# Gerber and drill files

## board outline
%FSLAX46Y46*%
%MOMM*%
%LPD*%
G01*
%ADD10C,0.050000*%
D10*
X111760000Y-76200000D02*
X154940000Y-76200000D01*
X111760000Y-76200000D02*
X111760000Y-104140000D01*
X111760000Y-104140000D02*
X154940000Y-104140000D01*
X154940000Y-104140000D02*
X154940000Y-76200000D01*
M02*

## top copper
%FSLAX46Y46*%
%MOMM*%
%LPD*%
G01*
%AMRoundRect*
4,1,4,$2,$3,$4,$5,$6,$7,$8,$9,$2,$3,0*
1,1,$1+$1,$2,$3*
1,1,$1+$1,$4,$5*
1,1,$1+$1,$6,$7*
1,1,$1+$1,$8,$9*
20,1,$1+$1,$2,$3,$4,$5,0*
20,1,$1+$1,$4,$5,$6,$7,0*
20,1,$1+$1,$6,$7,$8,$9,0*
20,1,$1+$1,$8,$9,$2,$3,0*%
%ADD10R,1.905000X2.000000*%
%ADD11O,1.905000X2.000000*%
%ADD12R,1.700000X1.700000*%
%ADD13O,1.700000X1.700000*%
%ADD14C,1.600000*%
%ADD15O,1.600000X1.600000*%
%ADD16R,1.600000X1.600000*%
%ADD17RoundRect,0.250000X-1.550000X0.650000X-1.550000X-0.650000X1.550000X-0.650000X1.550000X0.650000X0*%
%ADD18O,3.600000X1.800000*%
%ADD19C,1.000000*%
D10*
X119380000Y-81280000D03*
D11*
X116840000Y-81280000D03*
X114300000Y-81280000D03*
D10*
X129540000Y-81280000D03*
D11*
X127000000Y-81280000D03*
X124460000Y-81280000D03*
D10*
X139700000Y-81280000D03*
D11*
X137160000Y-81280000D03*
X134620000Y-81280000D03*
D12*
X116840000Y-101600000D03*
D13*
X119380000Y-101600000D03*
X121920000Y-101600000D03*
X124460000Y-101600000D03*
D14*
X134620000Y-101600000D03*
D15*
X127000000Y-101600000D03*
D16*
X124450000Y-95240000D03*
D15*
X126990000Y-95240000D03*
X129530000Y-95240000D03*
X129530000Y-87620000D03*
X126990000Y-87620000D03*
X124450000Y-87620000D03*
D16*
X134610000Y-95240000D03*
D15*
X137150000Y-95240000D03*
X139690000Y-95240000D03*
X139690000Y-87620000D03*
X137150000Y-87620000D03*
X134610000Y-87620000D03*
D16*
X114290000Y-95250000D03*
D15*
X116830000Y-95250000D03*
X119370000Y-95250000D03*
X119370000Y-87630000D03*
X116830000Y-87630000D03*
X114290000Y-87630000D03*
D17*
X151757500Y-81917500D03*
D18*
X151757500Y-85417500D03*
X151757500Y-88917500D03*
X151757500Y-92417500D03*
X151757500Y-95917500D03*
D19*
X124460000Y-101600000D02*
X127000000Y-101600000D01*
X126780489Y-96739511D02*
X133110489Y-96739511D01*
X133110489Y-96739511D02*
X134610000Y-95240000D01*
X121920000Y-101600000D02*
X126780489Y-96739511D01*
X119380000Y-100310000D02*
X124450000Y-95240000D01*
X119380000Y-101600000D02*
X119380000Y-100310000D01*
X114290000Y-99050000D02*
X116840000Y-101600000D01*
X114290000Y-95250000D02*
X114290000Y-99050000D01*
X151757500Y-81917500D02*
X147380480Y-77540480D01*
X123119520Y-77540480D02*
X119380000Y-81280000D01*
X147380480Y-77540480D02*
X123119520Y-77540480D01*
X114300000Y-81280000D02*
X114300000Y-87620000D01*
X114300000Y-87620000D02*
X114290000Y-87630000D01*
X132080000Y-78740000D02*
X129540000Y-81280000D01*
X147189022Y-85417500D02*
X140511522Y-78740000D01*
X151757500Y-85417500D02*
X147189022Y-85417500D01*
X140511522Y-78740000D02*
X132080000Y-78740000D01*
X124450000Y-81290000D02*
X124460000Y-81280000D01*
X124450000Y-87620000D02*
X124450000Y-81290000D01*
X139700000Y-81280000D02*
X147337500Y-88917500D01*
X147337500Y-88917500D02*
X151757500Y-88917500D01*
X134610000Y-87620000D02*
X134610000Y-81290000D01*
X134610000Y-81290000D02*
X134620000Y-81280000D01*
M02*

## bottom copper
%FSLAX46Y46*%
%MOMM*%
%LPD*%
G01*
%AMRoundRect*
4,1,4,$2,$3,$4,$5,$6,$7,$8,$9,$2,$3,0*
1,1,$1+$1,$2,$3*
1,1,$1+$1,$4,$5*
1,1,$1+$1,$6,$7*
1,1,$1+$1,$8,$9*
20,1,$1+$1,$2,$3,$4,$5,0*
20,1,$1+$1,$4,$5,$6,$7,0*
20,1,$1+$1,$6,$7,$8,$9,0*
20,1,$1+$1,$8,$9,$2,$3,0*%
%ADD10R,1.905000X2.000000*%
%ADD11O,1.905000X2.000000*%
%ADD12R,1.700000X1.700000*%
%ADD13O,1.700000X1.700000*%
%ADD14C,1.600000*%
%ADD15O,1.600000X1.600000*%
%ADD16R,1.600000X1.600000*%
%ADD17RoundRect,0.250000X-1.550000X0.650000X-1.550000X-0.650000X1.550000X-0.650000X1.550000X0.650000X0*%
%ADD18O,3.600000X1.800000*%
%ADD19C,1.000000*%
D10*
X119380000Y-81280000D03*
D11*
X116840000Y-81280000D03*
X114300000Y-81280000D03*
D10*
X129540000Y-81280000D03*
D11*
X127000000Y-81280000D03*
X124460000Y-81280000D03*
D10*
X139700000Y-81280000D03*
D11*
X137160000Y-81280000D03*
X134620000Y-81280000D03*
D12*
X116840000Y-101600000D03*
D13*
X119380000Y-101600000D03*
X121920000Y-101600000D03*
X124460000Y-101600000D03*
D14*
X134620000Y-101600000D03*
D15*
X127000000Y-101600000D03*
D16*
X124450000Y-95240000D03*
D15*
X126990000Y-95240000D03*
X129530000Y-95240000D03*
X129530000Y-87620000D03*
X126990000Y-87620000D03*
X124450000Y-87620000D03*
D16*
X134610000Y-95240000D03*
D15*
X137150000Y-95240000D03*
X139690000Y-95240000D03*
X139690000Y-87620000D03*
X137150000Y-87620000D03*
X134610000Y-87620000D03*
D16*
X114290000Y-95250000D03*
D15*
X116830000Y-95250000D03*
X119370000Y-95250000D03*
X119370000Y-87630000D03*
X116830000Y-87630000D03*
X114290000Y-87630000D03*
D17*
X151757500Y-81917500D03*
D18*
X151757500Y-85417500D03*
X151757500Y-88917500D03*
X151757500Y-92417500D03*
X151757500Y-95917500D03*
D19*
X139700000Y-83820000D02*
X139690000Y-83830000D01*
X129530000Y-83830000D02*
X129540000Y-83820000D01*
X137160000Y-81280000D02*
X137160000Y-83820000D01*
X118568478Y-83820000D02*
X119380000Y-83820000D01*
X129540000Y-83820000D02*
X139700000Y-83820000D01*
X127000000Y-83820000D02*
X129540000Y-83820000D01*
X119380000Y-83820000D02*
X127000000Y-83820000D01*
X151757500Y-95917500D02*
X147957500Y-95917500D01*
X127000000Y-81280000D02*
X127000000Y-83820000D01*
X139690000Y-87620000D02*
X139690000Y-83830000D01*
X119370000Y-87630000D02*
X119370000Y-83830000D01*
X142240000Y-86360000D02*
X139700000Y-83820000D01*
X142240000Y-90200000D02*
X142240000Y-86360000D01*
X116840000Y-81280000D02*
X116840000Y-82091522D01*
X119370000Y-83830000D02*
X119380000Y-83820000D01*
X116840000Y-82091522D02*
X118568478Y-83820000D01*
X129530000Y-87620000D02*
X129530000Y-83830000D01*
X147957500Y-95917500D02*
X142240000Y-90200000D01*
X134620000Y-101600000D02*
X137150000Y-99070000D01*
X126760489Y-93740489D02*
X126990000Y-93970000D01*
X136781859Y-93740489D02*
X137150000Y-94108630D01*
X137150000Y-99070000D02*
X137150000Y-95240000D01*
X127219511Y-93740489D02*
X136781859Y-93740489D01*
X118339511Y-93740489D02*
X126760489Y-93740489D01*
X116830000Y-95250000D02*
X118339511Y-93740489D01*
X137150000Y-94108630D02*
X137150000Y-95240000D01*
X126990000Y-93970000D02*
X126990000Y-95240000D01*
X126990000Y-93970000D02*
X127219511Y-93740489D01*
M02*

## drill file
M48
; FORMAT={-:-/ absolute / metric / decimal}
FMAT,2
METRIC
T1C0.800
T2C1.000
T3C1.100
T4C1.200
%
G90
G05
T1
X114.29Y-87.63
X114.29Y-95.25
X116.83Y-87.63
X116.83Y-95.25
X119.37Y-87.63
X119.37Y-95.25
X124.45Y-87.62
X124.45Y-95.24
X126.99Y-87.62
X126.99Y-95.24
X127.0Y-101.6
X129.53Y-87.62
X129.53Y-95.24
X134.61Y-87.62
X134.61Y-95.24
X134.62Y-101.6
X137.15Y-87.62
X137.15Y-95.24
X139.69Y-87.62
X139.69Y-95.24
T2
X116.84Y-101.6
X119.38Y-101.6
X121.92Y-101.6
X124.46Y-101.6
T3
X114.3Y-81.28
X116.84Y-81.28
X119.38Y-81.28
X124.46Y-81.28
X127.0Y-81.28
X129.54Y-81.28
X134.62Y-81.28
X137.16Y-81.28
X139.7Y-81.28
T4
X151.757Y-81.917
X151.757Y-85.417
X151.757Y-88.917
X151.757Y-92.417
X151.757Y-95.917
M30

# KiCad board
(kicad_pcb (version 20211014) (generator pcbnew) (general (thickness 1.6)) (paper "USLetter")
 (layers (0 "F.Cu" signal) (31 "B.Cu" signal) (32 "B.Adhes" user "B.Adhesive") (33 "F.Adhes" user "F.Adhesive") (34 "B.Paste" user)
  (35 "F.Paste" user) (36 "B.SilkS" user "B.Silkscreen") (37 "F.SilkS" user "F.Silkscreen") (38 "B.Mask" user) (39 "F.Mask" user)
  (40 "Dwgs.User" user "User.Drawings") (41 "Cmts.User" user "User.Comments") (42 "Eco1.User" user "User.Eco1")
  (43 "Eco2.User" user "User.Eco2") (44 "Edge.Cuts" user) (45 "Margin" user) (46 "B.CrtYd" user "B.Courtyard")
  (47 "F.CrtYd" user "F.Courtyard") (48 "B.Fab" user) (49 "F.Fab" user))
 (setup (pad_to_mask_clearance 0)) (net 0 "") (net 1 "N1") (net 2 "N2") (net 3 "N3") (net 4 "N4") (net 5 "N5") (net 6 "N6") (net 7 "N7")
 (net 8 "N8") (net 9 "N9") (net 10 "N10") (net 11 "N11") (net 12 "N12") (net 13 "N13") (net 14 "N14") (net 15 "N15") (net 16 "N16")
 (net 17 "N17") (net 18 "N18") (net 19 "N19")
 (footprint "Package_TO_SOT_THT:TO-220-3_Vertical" (layer "F.Cu") (at 119.38 81.28 180)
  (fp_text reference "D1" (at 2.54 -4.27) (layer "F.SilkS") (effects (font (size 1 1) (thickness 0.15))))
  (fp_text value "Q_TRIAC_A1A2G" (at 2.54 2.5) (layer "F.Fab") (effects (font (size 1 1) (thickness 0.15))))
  (pad "1" thru_hole rect locked (at 0 0 180) (size 1.905 2) (drill 1.1) (layers *.Cu *.Mask) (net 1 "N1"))
  (pad "2" thru_hole oval locked (at 2.54 0 180) (size 1.905 2) (drill 1.1) (layers *.Cu *.Mask) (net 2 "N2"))
  (pad "3" thru_hole oval locked (at 5.08 0 180) (size 1.905 2) (drill 1.1) (layers *.Cu *.Mask) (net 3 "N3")))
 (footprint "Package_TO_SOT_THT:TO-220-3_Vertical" (layer "F.Cu") (at 129.54 81.28 180)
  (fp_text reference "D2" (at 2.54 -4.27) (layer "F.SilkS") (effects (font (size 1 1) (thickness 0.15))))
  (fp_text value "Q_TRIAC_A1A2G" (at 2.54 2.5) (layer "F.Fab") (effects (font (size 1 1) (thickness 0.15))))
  (pad "1" thru_hole rect locked (at 0 0 180) (size 1.905 2) (drill 1.1) (layers *.Cu *.Mask) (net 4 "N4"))
  (pad "2" thru_hole oval locked (at 2.54 0 180) (size 1.905 2) (drill 1.1) (layers *.Cu *.Mask) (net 2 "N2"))
  (pad "3" thru_hole oval locked (at 5.08 0 180) (size 1.905 2) (drill 1.1) (layers *.Cu *.Mask) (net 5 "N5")))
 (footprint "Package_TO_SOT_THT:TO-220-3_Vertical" (layer "F.Cu") (at 139.7 81.28 180)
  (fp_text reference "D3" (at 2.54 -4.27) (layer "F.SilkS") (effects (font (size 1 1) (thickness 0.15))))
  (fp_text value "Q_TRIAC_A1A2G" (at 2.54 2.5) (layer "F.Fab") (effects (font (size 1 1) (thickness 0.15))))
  (pad "1" thru_hole rect locked (at 0 0 180) (size 1.905 2) (drill 1.1) (layers *.Cu *.Mask) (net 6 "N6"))
  (pad "2" thru_hole oval locked (at 2.54 0 180) (size 1.905 2) (drill 1.1) (layers *.Cu *.Mask) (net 2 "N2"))
  (pad "3" thru_hole oval locked (at 5.08 0 180) (size 1.905 2) (drill 1.1) (layers *.Cu *.Mask) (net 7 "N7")))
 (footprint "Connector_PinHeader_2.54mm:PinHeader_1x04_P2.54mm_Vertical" (layer "F.Cu") (at 116.84 101.6 90)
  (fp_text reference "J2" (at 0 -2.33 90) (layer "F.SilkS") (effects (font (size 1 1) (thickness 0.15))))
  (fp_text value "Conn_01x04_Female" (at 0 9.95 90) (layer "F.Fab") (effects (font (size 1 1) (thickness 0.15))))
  (pad "1" thru_hole rect locked (at 0 0 90) (size 1.7 1.7) (drill 1) (layers *.Cu *.Mask) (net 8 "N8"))
  (pad "2" thru_hole oval locked (at 0 2.54 90) (size 1.7 1.7) (drill 1) (layers *.Cu *.Mask) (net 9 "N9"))
  (pad "3" thru_hole oval locked (at 0 5.08 90) (size 1.7 1.7) (drill 1) (layers *.Cu *.Mask) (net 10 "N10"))
  (pad "4" thru_hole oval locked (at 0 7.62 90) (size 1.7 1.7) (drill 1) (layers *.Cu *.Mask) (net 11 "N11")))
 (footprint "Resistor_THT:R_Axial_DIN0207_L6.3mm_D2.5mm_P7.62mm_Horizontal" (layer "F.Cu") (at 134.62 101.6 180)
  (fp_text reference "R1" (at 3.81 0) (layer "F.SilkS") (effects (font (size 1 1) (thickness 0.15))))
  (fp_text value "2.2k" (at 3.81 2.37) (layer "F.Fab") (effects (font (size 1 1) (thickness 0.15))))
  (pad "1" thru_hole circle locked (at 0 0 180) (size 1.6 1.6) (drill 0.8) (layers *.Cu *.Mask) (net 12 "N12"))
  (pad "2" thru_hole oval locked (at 7.62 0 180) (size 1.6 1.6) (drill 0.8) (layers *.Cu *.Mask) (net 11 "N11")))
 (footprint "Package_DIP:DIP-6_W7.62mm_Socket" (layer "F.Cu") (at 124.45 95.24 90)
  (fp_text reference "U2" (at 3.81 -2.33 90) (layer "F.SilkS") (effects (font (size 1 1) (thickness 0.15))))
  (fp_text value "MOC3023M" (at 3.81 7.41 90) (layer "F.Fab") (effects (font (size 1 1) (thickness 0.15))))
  (pad "1" thru_hole rect locked (at 0 0 90) (size 1.6 1.6) (drill 0.8) (layers *.Cu *.Mask) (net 9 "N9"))
  (pad "2" thru_hole oval locked (at 0 2.54 90) (size 1.6 1.6) (drill 0.8) (layers *.Cu *.Mask) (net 12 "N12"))
  (pad "3" thru_hole oval locked (at 0 5.08 90) (size 1.6 1.6) (drill 0.8) (layers *.Cu *.Mask) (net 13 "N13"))
  (pad "4" thru_hole oval locked (at 7.62 5.08 90) (size 1.6 1.6) (drill 0.8) (layers *.Cu *.Mask) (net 2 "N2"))
  (pad "5" thru_hole oval locked (at 7.62 2.54 90) (size 1.6 1.6) (drill 0.8) (layers *.Cu *.Mask) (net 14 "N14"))
  (pad "6" thru_hole oval locked (at 7.62 0 90) (size 1.6 1.6) (drill 0.8) (layers *.Cu *.Mask) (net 5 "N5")))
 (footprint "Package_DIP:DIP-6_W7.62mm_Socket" (layer "F.Cu") (at 134.61 95.24 90)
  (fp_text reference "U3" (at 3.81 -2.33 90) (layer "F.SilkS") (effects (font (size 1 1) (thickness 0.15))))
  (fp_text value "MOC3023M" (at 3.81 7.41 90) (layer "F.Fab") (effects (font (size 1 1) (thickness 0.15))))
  (pad "1" thru_hole rect locked (at 0 0 90) (size 1.6 1.6) (drill 0.8) (layers *.Cu *.Mask) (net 10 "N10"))
  (pad "2" thru_hole oval locked (at 0 2.54 90) (size 1.6 1.6) (drill 0.8) (layers *.Cu *.Mask) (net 12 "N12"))
  (pad "3" thru_hole oval locked (at 0 5.08 90) (size 1.6 1.6) (drill 0.8) (layers *.Cu *.Mask) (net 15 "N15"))
  (pad "4" thru_hole oval locked (at 7.62 5.08 90) (size 1.6 1.6) (drill 0.8) (layers *.Cu *.Mask) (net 2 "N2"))
  (pad "5" thru_hole oval locked (at 7.62 2.54 90) (size 1.6 1.6) (drill 0.8) (layers *.Cu *.Mask) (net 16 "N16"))
  (pad "6" thru_hole oval locked (at 7.62 0 90) (size 1.6 1.6) (drill 0.8) (layers *.Cu *.Mask) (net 7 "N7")))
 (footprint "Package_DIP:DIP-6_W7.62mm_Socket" (layer "F.Cu") (at 114.29 95.25 90)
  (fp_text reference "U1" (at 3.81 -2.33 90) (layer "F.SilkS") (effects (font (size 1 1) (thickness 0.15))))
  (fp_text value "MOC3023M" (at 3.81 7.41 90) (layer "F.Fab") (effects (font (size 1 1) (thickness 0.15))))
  (pad "1" thru_hole rect locked (at 0 0 90) (size 1.6 1.6) (drill 0.8) (layers *.Cu *.Mask) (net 8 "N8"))
  (pad "2" thru_hole oval locked (at 0 2.54 90) (size 1.6 1.6) (drill 0.8) (layers *.Cu *.Mask) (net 12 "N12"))
  (pad "3" thru_hole oval locked (at 0 5.08 90) (size 1.6 1.6) (drill 0.8) (layers *.Cu *.Mask) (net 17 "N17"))
  (pad "4" thru_hole oval locked (at 7.62 5.08 90) (size 1.6 1.6) (drill 0.8) (layers *.Cu *.Mask) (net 2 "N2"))
  (pad "5" thru_hole oval locked (at 7.62 2.54 90) (size 1.6 1.6) (drill 0.8) (layers *.Cu *.Mask) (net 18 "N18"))
  (pad "6" thru_hole oval locked (at 7.62 0 90) (size 1.6 1.6) (drill 0.8) (layers *.Cu *.Mask) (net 3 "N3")))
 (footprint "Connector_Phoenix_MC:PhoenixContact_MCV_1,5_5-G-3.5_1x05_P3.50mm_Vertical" (layer "F.Cu") (at 151.7575 81.9175 -90)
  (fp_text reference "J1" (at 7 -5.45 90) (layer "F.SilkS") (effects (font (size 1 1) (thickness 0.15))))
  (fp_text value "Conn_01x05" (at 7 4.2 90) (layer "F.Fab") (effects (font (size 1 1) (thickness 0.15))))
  (pad "1" thru_hole roundrect locked (at 0 0 270) (size 1.8 3.6) (drill 1.2) (layers *.Cu *.Mask) (roundrect_rratio 0.138889) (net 1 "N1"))
  (pad "2" thru_hole oval locked (at 3.5 0 270) (size 1.8 3.6) (drill 1.2) (layers *.Cu *.Mask) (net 4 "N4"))
  (pad "3" thru_hole oval locked (at 7 0 270) (size 1.8 3.6) (drill 1.2) (layers *.Cu *.Mask) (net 6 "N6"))
  (pad "4" thru_hole oval locked (at 10.5 0 270) (size 1.8 3.6) (drill 1.2) (layers *.Cu *.Mask) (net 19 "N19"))
  (pad "5" thru_hole oval locked (at 14 0 270) (size 1.8 3.6) (drill 1.2) (layers *.Cu *.Mask) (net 2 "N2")))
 (gr_line (start 111.76 76.2) (end 154.94 76.2) (layer "Edge.Cuts") (width 0.05))
 (gr_line (start 111.76 76.2) (end 111.76 104.14) (layer "Edge.Cuts") (width 0.05))
 (gr_line (start 111.76 104.14) (end 154.94 104.14) (layer "Edge.Cuts") (width 0.05))
 (gr_line (start 154.94 104.14) (end 154.94 76.2) (layer "Edge.Cuts") (width 0.05))
 (segment (start 139.7 83.82) (end 139.69 83.83) (width 1) (layer "B.Cu") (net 2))
 (segment (start 129.53 83.83) (end 129.54 83.82) (width 1) (layer "B.Cu") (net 2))
 (segment (start 137.16 81.28) (end 137.16 83.82) (width 1) (layer "B.Cu") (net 2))
 (segment (start 118.568478 83.82) (end 119.38 83.82) (width 1) (layer "B.Cu") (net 2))
 (segment (start 129.54 83.82) (end 139.7 83.82) (width 1) (layer "B.Cu") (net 2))
 (segment (start 127 83.82) (end 129.54 83.82) (width 1) (layer "B.Cu") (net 2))
 (segment (start 119.38 83.82) (end 127 83.82) (width 1) (layer "B.Cu") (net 2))
 (segment (start 151.7575 95.9175) (end 147.9575 95.9175) (width 1) (layer "B.Cu") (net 2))
 (segment (start 127 81.28) (end 127 83.82) (width 1) (layer "B.Cu") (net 2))
 (segment (start 139.69 87.62) (end 139.69 83.83) (width 1) (layer "B.Cu") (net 2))
 (segment (start 119.37 87.63) (end 119.37 83.83) (width 1) (layer "B.Cu") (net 2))
 (segment (start 142.24 86.36) (end 139.7 83.82) (width 1) (layer "B.Cu") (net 2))
 (segment (start 142.24 90.2) (end 142.24 86.36) (width 1) (layer "B.Cu") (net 2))
 (segment (start 116.84 81.28) (end 116.84 82.091522) (width 1) (layer "B.Cu") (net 2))
 (segment (start 119.37 83.83) (end 119.38 83.82) (width 1) (layer "B.Cu") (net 2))
 (segment (start 116.84 82.091522) (end 118.568478 83.82) (width 1) (layer "B.Cu") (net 2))
 (segment (start 129.53 87.62) (end 129.53 83.83) (width 1) (layer "B.Cu") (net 2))
 (segment (start 147.9575 95.9175) (end 142.24 90.2) (width 1) (layer "B.Cu") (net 2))
 (segment (start 124.46 101.6) (end 127 101.6) (width 1) (layer "F.Cu") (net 11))
 (segment (start 126.780489 96.739511) (end 133.110489 96.739511) (width 1) (layer "F.Cu") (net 10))
 (segment (start 133.110489 96.739511) (end 134.61 95.24) (width 1) (layer "F.Cu") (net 10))
 (segment (start 121.92 101.6) (end 126.780489 96.739511) (width 1) (layer "F.Cu") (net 10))
 (segment (start 119.38 100.31) (end 124.45 95.24) (width 1) (layer "F.Cu") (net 9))
 (segment (start 119.38 101.6) (end 119.38 100.31) (width 1) (layer "F.Cu") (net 9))
 (segment (start 114.29 99.05) (end 116.84 101.6) (width 1) (layer "F.Cu") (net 8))
 (segment (start 114.29 95.25) (end 114.29 99.05) (width 1) (layer "F.Cu") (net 8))
 (segment (start 134.62 101.6) (end 137.15 99.07) (width 1) (layer "B.Cu") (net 12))
 (segment (start 126.760489 93.740489) (end 126.99 93.97) (width 1) (layer "B.Cu") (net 12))
 (segment (start 136.781859 93.740489) (end 137.15 94.10863) (width 1) (layer "B.Cu") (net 12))
 (segment (start 137.15 99.07) (end 137.15 95.24) (width 1) (layer "B.Cu") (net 12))
 (segment (start 127.219511 93.740489) (end 136.781859 93.740489) (width 1) (layer "B.Cu") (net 12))
 (segment (start 118.339511 93.740489) (end 126.760489 93.740489) (width 1) (layer "B.Cu") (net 12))
 (segment (start 116.83 95.25) (end 118.339511 93.740489) (width 1) (layer "B.Cu") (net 12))
 (segment (start 137.15 94.10863) (end 137.15 95.24) (width 1) (layer "B.Cu") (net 12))
 (segment (start 126.99 93.97) (end 126.99 95.24) (width 1) (layer "B.Cu") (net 12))
 (segment (start 126.99 93.97) (end 127.219511 93.740489) (width 1) (layer "B.Cu") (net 12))
 (segment (start 151.7575 81.9175) (end 147.38048 77.54048) (width 1) (layer "F.Cu") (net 1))
 (segment (start 123.11952 77.54048) (end 119.38 81.28) (width 1) (layer "F.Cu") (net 1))
 (segment (start 147.38048 77.54048) (end 123.11952 77.54048) (width 1) (layer "F.Cu") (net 1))
 (segment (start 114.3 81.28) (end 114.3 87.62) (width 1) (layer "F.Cu") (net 3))
 (segment (start 114.3 87.62) (end 114.29 87.63) (width 1) (layer "F.Cu") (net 3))
 (segment (start 132.08 78.74) (end 129.54 81.28) (width 1) (layer "F.Cu") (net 4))
 (segment (start 147.189022 85.4175) (end 140.511522 78.74) (width 1) (layer "F.Cu") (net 4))
 (segment (start 151.7575 85.4175) (end 147.189022 85.4175) (width 1) (layer "F.Cu") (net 4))
 (segment (start 140.511522 78.74) (end 132.08 78.74) (width 1) (layer "F.Cu") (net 4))
 (segment (start 124.45 81.29) (end 124.46 81.28) (width 1) (layer "F.Cu") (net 5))
 (segment (start 124.45 87.62) (end 124.45 81.29) (width 1) (layer "F.Cu") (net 5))
 (segment (start 139.7 81.28) (end 147.3375 88.9175) (width 1) (layer "F.Cu") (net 6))
 (segment (start 147.3375 88.9175) (end 151.7575 88.9175) (width 1) (layer "F.Cu") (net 6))
 (segment (start 134.61 87.62) (end 134.61 81.29) (width 1) (layer "F.Cu") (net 7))
 (segment (start 134.61 81.29) (end 134.62 81.28) (width 1) (layer "F.Cu") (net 7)))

